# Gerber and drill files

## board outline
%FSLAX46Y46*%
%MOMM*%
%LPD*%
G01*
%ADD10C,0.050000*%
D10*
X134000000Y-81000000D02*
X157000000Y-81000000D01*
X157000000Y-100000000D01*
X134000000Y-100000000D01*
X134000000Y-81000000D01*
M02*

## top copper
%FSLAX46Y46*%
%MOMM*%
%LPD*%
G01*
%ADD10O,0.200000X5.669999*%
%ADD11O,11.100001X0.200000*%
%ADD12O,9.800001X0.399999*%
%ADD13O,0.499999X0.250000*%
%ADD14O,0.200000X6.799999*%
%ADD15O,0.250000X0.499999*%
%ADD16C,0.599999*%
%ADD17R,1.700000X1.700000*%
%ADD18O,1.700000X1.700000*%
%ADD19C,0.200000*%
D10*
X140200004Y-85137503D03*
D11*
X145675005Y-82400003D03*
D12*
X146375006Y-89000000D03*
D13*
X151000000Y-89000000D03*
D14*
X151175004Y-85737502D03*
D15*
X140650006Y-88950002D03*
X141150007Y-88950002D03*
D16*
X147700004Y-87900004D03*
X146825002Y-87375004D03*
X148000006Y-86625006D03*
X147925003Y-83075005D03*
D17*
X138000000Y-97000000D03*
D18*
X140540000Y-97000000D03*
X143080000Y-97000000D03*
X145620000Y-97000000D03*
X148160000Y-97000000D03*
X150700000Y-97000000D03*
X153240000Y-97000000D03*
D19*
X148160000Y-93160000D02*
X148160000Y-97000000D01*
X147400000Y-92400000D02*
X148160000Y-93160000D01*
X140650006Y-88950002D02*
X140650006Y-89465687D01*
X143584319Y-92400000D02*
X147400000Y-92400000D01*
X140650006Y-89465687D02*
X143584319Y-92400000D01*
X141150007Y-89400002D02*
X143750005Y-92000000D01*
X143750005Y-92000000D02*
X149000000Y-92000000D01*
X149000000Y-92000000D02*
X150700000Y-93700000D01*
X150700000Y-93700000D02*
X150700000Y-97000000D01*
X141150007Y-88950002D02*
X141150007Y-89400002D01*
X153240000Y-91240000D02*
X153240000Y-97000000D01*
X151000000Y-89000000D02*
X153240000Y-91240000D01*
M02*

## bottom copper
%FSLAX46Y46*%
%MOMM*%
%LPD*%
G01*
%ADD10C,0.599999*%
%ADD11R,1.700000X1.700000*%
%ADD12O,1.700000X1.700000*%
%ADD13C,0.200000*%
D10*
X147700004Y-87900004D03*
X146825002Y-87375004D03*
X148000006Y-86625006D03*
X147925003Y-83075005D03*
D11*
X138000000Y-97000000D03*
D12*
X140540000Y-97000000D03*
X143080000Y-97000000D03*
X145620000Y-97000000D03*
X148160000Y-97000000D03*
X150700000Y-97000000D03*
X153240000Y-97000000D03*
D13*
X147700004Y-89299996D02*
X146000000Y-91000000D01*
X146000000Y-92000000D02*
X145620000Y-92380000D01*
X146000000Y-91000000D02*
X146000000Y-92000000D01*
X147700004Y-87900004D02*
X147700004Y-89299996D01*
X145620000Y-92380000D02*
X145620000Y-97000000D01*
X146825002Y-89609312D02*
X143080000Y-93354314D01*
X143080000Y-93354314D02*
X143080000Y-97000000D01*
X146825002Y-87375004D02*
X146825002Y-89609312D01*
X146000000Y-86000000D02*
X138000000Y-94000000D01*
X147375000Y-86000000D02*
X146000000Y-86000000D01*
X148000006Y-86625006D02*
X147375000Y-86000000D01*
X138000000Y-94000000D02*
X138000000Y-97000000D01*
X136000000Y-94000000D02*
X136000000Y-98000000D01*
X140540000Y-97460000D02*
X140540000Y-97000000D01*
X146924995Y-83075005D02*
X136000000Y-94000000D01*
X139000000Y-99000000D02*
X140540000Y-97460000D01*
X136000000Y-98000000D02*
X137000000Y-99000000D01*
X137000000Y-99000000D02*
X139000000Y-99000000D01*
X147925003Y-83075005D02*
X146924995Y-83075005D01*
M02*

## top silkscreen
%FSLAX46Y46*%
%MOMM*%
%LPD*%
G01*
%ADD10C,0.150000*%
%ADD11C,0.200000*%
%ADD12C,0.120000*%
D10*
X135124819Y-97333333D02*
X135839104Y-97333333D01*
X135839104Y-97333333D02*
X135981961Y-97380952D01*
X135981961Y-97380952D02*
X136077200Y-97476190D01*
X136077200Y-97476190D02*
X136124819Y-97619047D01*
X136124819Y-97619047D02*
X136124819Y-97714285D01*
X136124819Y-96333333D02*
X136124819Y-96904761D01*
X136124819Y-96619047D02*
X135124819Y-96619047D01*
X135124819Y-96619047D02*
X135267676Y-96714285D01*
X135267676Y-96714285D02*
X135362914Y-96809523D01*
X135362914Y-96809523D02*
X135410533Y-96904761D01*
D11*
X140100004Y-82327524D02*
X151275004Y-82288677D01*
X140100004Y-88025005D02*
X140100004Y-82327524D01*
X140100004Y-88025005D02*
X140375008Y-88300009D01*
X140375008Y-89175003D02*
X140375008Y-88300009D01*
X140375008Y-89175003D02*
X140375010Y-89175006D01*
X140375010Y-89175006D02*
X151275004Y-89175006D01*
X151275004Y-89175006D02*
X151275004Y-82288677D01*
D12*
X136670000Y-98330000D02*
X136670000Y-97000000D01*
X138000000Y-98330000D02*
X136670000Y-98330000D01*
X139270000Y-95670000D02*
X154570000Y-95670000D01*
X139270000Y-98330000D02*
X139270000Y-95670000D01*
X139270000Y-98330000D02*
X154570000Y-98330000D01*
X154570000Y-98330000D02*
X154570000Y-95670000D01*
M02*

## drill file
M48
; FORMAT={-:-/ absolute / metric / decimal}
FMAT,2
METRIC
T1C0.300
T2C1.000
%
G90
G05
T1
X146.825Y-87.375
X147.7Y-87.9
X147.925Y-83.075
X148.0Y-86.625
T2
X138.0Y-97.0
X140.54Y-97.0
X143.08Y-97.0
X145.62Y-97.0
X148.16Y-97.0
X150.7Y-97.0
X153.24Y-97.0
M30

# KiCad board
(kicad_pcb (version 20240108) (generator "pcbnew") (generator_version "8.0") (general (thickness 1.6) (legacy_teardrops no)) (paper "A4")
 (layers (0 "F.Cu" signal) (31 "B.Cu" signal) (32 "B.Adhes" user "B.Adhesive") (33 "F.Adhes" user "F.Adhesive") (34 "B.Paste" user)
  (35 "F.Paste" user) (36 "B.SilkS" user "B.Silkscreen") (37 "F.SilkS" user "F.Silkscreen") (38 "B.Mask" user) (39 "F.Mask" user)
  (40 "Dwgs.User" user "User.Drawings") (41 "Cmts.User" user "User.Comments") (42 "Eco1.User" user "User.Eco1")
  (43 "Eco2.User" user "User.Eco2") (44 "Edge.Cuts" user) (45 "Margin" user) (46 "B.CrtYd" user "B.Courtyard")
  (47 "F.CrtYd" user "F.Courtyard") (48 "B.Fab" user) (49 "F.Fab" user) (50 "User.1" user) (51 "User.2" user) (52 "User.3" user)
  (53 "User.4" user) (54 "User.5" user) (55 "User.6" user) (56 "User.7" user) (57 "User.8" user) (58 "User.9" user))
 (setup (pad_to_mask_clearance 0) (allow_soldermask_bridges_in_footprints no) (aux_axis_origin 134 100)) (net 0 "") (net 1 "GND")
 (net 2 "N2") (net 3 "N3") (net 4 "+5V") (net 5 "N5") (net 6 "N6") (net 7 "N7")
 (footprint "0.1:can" (layer "F.Cu") (at 140.000007 89.275003)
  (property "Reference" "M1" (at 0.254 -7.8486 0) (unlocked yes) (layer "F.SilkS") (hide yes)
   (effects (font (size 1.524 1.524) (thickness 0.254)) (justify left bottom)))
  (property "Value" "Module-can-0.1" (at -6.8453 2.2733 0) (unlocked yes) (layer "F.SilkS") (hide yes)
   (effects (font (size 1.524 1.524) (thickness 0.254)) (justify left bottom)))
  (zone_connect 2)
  (fp_line (start 0.099997 -6.947479) (end 11.274997 -6.986326) (stroke (width 0.2) (type solid)) (layer "F.SilkS"))
  (fp_line (start 0.099997 -1.249998) (end 0.099997 -6.947479) (stroke (width 0.2) (type solid)) (layer "F.SilkS"))
  (fp_line (start 0.099997 -1.249998) (end 0.375001 -0.974994) (stroke (width 0.2) (type solid)) (layer "F.SilkS"))
  (fp_line (start 0.375001 -0.1) (end 0.375001 -0.974994) (stroke (width 0.2) (type solid)) (layer "F.SilkS"))
  (fp_line (start 0.375001 -0.1) (end 0.375003 -0.099997) (stroke (width 0.2) (type solid)) (layer "F.SilkS"))
  (fp_line (start 0.375003 -0.099997) (end 11.274997 -0.099997) (stroke (width 0.2) (type solid)) (layer "F.SilkS"))
  (fp_line (start 11.274997 -0.099997) (end 11.274997 -6.986326) (stroke (width 0.2) (type solid)) (layer "F.SilkS"))
  (pad "E1" smd oval (at 0.199997 -4.1375 180) (size 0.2 5.669999) (layers "F.Cu" "F.Paste") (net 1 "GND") (solder_mask_margin 0.1016)
   (solder_paste_margin -49.999999) (zone_connect 2))
  (pad "E1" smd oval (at 5.674998 -6.875 90) (size 0.2 11.100001) (layers "F.Cu" "F.Paste") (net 1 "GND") (solder_mask_margin 0.1016)
   (solder_paste_margin -49.999999) (zone_connect 2))
  (pad "E1" smd oval (at 6.374999 -0.275003 270) (size 0.399999 9.800001) (layers "F.Cu" "F.Paste") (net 1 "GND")
   (solder_mask_margin 0.1016) (solder_paste_margin -49.999999) (zone_connect 2))
  (pad "E1" smd oval (at 10.999993 -0.275003 180) (size 0.499999 0.25) (layers "F.Cu" "F.Paste" "F.Mask") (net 1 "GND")
   (solder_paste_margin -49.999999) (zone_connect 2))
  (pad "E1" smd oval (at 11.174997 -3.537501 180) (size 0.2 6.799999) (layers "F.Cu" "F.Paste") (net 1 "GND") (solder_mask_margin 0.1016)
   (solder_paste_margin -49.999999) (zone_connect 2))
  (pad "S1" smd oval (at 0.649999 -0.325001) (size 0.25 0.499999) (layers "F.Cu" "F.Paste" "F.Mask") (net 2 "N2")
   (solder_paste_margin -49.999999) (zone_connect 2))
  (pad "S2" smd oval (at 1.15 -0.325001) (size 0.25 0.499999) (layers "F.Cu" "F.Paste" "F.Mask") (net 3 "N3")
   (solder_paste_margin -49.999999) (zone_connect 2))
  (pad "V1" thru_hole circle (at 7.699997 -1.374999 180) (size 0.599999 0.599999) (drill 0.299999) (layers "*.Cu" "*.Mask")
   (remove_unused_layers no) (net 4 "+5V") (solder_paste_margin -49.999999) (zone_connect 2))
  (pad "V2" thru_hole circle (at 6.824995 -1.899999 180) (size 0.599999 0.599999) (drill 0.299999) (layers "*.Cu" "*.Mask")
   (remove_unused_layers no) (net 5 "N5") (solder_paste_margin -49.999999) (zone_connect 2))
  (pad "V5" thru_hole circle (at 7.999999 -2.649997 270) (size 0.599999 0.599999) (drill 0.299999) (layers "*.Cu" "*.Mask")
   (remove_unused_layers no) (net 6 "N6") (solder_paste_margin -49.999999) (zone_connect 2))
  (pad "V6" thru_hole circle (at 7.924996 -6.199998 270) (size 0.599999 0.599999) (drill 0.299999) (layers "*.Cu" "*.Mask")
   (remove_unused_layers no) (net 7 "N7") (solder_paste_margin -49.999999) (zone_connect 2))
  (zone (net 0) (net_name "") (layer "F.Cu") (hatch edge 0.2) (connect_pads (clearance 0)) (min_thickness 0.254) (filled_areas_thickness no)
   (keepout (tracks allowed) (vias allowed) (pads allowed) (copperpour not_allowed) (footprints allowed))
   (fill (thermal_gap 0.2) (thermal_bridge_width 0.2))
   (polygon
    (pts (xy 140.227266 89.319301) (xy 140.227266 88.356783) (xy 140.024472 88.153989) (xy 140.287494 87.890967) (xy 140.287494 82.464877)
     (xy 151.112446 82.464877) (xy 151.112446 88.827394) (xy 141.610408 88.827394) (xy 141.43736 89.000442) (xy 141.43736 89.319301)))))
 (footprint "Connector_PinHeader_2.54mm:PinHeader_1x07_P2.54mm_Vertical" (layer "F.Cu") (at 138 97 90)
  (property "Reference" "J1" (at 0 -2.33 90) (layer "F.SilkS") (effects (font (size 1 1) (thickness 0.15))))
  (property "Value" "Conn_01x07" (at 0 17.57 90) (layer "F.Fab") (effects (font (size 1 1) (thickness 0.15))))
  (fp_line (start -1.33 -1.33) (end 0 -1.33) (stroke (width 0.12) (type solid)) (layer "F.SilkS"))
  (fp_line (start -1.33 0) (end -1.33 -1.33) (stroke (width 0.12) (type solid)) (layer "F.SilkS"))
  (fp_line (start 1.33 1.27) (end 1.33 16.57) (stroke (width 0.12) (type solid)) (layer "F.SilkS"))
  (fp_line (start -1.33 1.27) (end 1.33 1.27) (stroke (width 0.12) (type solid)) (layer "F.SilkS"))
  (fp_line (start -1.33 1.27) (end -1.33 16.57) (stroke (width 0.12) (type solid)) (layer "F.SilkS"))
  (fp_line (start -1.33 16.57) (end 1.33 16.57) (stroke (width 0.12) (type solid)) (layer "F.SilkS"))
  (pad "1" thru_hole rect (at 0 0 90) (size 1.7 1.7) (drill 1) (layers "*.Cu" "*.Mask") (remove_unused_layers no) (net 6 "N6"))
  (pad "2" thru_hole oval (at 0 2.54 90) (size 1.7 1.7) (drill 1) (layers "*.Cu" "*.Mask") (remove_unused_layers no) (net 7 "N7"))
  (pad "3" thru_hole oval (at 0 5.08 90) (size 1.7 1.7) (drill 1) (layers "*.Cu" "*.Mask") (remove_unused_layers no) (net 5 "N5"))
  (pad "4" thru_hole oval (at 0 7.62 90) (size 1.7 1.7) (drill 1) (layers "*.Cu" "*.Mask") (remove_unused_layers no) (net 4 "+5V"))
  (pad "5" thru_hole oval (at 0 10.16 90) (size 1.7 1.7) (drill 1) (layers "*.Cu" "*.Mask") (remove_unused_layers no) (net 2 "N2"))
  (pad "6" thru_hole oval (at 0 12.7 90) (size 1.7 1.7) (drill 1) (layers "*.Cu" "*.Mask") (remove_unused_layers no) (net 3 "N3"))
  (pad "7" thru_hole oval (at 0 15.24 90) (size 1.7 1.7) (drill 1) (layers "*.Cu" "*.Mask") (remove_unused_layers no) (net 1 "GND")))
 (gr_rect (start 134 81) (end 157 100) (stroke (width 0.05) (type default)) (fill none) (layer "Edge.Cuts"))
 (segment (start 147.700004 89.299996) (end 146 91) (width 0.2) (layer "B.Cu") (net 4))
 (segment (start 146 92) (end 145.62 92.38) (width 0.2) (layer "B.Cu") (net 4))
 (segment (start 146 91) (end 146 92) (width 0.2) (layer "B.Cu") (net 4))
 (segment (start 147.700004 87.900004) (end 147.700004 89.299996) (width 0.2) (layer "B.Cu") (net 4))
 (segment (start 145.62 92.38) (end 145.62 97) (width 0.2) (layer "B.Cu") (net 4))
 (segment (start 146.825002 89.609312) (end 143.08 93.354314) (width 0.2) (layer "B.Cu") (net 5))
 (segment (start 143.08 93.354314) (end 143.08 97) (width 0.2) (layer "B.Cu") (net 5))
 (segment (start 146.825002 87.375004) (end 146.825002 89.609312) (width 0.2) (layer "B.Cu") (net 5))
 (segment (start 148.16 93.16) (end 148.16 97) (width 0.2) (layer "F.Cu") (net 2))
 (segment (start 147.4 92.4) (end 148.16 93.16) (width 0.2) (layer "F.Cu") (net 2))
 (segment (start 140.650006 88.950002) (end 140.650006 89.465687) (width 0.2) (layer "F.Cu") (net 2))
 (segment (start 143.584319 92.4) (end 147.4 92.4) (width 0.2) (layer "F.Cu") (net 2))
 (segment (start 140.650006 89.465687) (end 143.584319 92.4) (width 0.2) (layer "F.Cu") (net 2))
 (segment (start 141.150007 89.400002) (end 143.750005 92) (width 0.2) (layer "F.Cu") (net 3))
 (segment (start 143.750005 92) (end 149 92) (width 0.2) (layer "F.Cu") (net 3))
 (segment (start 149 92) (end 150.7 93.7) (width 0.2) (layer "F.Cu") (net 3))
 (segment (start 150.7 93.7) (end 150.7 97) (width 0.2) (layer "F.Cu") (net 3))
 (segment (start 141.150007 88.950002) (end 141.150007 89.400002) (width 0.2) (layer "F.Cu") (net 3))
 (segment (start 146 86) (end 138 94) (width 0.2) (layer "B.Cu") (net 6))
 (segment (start 147.375 86) (end 146 86) (width 0.2) (layer "B.Cu") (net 6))
 (segment (start 148.000006 86.625006) (end 147.375 86) (width 0.2) (layer "B.Cu") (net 6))
 (segment (start 138 94) (end 138 97) (width 0.2) (layer "B.Cu") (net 6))
 (segment (start 153.24 91.24) (end 153.24 97) (width 0.2) (layer "F.Cu") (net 1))
 (segment (start 151 89) (end 153.24 91.24) (width 0.2) (layer "F.Cu") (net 1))
 (segment (start 136 94) (end 136 98) (width 0.2) (layer "B.Cu") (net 7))
 (segment (start 140.54 97.46) (end 140.54 97) (width 0.2) (layer "B.Cu") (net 7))
 (segment (start 146.924995 83.075005) (end 136 94) (width 0.2) (layer "B.Cu") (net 7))
 (segment (start 139 99) (end 140.54 97.46) (width 0.2) (layer "B.Cu") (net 7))
 (segment (start 136 98) (end 137 99) (width 0.2) (layer "B.Cu") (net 7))
 (segment (start 137 99) (end 139 99) (width 0.2) (layer "B.Cu") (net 7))
 (segment (start 147.925003 83.075005) (end 146.924995 83.075005) (width 0.2) (layer "B.Cu") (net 7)))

